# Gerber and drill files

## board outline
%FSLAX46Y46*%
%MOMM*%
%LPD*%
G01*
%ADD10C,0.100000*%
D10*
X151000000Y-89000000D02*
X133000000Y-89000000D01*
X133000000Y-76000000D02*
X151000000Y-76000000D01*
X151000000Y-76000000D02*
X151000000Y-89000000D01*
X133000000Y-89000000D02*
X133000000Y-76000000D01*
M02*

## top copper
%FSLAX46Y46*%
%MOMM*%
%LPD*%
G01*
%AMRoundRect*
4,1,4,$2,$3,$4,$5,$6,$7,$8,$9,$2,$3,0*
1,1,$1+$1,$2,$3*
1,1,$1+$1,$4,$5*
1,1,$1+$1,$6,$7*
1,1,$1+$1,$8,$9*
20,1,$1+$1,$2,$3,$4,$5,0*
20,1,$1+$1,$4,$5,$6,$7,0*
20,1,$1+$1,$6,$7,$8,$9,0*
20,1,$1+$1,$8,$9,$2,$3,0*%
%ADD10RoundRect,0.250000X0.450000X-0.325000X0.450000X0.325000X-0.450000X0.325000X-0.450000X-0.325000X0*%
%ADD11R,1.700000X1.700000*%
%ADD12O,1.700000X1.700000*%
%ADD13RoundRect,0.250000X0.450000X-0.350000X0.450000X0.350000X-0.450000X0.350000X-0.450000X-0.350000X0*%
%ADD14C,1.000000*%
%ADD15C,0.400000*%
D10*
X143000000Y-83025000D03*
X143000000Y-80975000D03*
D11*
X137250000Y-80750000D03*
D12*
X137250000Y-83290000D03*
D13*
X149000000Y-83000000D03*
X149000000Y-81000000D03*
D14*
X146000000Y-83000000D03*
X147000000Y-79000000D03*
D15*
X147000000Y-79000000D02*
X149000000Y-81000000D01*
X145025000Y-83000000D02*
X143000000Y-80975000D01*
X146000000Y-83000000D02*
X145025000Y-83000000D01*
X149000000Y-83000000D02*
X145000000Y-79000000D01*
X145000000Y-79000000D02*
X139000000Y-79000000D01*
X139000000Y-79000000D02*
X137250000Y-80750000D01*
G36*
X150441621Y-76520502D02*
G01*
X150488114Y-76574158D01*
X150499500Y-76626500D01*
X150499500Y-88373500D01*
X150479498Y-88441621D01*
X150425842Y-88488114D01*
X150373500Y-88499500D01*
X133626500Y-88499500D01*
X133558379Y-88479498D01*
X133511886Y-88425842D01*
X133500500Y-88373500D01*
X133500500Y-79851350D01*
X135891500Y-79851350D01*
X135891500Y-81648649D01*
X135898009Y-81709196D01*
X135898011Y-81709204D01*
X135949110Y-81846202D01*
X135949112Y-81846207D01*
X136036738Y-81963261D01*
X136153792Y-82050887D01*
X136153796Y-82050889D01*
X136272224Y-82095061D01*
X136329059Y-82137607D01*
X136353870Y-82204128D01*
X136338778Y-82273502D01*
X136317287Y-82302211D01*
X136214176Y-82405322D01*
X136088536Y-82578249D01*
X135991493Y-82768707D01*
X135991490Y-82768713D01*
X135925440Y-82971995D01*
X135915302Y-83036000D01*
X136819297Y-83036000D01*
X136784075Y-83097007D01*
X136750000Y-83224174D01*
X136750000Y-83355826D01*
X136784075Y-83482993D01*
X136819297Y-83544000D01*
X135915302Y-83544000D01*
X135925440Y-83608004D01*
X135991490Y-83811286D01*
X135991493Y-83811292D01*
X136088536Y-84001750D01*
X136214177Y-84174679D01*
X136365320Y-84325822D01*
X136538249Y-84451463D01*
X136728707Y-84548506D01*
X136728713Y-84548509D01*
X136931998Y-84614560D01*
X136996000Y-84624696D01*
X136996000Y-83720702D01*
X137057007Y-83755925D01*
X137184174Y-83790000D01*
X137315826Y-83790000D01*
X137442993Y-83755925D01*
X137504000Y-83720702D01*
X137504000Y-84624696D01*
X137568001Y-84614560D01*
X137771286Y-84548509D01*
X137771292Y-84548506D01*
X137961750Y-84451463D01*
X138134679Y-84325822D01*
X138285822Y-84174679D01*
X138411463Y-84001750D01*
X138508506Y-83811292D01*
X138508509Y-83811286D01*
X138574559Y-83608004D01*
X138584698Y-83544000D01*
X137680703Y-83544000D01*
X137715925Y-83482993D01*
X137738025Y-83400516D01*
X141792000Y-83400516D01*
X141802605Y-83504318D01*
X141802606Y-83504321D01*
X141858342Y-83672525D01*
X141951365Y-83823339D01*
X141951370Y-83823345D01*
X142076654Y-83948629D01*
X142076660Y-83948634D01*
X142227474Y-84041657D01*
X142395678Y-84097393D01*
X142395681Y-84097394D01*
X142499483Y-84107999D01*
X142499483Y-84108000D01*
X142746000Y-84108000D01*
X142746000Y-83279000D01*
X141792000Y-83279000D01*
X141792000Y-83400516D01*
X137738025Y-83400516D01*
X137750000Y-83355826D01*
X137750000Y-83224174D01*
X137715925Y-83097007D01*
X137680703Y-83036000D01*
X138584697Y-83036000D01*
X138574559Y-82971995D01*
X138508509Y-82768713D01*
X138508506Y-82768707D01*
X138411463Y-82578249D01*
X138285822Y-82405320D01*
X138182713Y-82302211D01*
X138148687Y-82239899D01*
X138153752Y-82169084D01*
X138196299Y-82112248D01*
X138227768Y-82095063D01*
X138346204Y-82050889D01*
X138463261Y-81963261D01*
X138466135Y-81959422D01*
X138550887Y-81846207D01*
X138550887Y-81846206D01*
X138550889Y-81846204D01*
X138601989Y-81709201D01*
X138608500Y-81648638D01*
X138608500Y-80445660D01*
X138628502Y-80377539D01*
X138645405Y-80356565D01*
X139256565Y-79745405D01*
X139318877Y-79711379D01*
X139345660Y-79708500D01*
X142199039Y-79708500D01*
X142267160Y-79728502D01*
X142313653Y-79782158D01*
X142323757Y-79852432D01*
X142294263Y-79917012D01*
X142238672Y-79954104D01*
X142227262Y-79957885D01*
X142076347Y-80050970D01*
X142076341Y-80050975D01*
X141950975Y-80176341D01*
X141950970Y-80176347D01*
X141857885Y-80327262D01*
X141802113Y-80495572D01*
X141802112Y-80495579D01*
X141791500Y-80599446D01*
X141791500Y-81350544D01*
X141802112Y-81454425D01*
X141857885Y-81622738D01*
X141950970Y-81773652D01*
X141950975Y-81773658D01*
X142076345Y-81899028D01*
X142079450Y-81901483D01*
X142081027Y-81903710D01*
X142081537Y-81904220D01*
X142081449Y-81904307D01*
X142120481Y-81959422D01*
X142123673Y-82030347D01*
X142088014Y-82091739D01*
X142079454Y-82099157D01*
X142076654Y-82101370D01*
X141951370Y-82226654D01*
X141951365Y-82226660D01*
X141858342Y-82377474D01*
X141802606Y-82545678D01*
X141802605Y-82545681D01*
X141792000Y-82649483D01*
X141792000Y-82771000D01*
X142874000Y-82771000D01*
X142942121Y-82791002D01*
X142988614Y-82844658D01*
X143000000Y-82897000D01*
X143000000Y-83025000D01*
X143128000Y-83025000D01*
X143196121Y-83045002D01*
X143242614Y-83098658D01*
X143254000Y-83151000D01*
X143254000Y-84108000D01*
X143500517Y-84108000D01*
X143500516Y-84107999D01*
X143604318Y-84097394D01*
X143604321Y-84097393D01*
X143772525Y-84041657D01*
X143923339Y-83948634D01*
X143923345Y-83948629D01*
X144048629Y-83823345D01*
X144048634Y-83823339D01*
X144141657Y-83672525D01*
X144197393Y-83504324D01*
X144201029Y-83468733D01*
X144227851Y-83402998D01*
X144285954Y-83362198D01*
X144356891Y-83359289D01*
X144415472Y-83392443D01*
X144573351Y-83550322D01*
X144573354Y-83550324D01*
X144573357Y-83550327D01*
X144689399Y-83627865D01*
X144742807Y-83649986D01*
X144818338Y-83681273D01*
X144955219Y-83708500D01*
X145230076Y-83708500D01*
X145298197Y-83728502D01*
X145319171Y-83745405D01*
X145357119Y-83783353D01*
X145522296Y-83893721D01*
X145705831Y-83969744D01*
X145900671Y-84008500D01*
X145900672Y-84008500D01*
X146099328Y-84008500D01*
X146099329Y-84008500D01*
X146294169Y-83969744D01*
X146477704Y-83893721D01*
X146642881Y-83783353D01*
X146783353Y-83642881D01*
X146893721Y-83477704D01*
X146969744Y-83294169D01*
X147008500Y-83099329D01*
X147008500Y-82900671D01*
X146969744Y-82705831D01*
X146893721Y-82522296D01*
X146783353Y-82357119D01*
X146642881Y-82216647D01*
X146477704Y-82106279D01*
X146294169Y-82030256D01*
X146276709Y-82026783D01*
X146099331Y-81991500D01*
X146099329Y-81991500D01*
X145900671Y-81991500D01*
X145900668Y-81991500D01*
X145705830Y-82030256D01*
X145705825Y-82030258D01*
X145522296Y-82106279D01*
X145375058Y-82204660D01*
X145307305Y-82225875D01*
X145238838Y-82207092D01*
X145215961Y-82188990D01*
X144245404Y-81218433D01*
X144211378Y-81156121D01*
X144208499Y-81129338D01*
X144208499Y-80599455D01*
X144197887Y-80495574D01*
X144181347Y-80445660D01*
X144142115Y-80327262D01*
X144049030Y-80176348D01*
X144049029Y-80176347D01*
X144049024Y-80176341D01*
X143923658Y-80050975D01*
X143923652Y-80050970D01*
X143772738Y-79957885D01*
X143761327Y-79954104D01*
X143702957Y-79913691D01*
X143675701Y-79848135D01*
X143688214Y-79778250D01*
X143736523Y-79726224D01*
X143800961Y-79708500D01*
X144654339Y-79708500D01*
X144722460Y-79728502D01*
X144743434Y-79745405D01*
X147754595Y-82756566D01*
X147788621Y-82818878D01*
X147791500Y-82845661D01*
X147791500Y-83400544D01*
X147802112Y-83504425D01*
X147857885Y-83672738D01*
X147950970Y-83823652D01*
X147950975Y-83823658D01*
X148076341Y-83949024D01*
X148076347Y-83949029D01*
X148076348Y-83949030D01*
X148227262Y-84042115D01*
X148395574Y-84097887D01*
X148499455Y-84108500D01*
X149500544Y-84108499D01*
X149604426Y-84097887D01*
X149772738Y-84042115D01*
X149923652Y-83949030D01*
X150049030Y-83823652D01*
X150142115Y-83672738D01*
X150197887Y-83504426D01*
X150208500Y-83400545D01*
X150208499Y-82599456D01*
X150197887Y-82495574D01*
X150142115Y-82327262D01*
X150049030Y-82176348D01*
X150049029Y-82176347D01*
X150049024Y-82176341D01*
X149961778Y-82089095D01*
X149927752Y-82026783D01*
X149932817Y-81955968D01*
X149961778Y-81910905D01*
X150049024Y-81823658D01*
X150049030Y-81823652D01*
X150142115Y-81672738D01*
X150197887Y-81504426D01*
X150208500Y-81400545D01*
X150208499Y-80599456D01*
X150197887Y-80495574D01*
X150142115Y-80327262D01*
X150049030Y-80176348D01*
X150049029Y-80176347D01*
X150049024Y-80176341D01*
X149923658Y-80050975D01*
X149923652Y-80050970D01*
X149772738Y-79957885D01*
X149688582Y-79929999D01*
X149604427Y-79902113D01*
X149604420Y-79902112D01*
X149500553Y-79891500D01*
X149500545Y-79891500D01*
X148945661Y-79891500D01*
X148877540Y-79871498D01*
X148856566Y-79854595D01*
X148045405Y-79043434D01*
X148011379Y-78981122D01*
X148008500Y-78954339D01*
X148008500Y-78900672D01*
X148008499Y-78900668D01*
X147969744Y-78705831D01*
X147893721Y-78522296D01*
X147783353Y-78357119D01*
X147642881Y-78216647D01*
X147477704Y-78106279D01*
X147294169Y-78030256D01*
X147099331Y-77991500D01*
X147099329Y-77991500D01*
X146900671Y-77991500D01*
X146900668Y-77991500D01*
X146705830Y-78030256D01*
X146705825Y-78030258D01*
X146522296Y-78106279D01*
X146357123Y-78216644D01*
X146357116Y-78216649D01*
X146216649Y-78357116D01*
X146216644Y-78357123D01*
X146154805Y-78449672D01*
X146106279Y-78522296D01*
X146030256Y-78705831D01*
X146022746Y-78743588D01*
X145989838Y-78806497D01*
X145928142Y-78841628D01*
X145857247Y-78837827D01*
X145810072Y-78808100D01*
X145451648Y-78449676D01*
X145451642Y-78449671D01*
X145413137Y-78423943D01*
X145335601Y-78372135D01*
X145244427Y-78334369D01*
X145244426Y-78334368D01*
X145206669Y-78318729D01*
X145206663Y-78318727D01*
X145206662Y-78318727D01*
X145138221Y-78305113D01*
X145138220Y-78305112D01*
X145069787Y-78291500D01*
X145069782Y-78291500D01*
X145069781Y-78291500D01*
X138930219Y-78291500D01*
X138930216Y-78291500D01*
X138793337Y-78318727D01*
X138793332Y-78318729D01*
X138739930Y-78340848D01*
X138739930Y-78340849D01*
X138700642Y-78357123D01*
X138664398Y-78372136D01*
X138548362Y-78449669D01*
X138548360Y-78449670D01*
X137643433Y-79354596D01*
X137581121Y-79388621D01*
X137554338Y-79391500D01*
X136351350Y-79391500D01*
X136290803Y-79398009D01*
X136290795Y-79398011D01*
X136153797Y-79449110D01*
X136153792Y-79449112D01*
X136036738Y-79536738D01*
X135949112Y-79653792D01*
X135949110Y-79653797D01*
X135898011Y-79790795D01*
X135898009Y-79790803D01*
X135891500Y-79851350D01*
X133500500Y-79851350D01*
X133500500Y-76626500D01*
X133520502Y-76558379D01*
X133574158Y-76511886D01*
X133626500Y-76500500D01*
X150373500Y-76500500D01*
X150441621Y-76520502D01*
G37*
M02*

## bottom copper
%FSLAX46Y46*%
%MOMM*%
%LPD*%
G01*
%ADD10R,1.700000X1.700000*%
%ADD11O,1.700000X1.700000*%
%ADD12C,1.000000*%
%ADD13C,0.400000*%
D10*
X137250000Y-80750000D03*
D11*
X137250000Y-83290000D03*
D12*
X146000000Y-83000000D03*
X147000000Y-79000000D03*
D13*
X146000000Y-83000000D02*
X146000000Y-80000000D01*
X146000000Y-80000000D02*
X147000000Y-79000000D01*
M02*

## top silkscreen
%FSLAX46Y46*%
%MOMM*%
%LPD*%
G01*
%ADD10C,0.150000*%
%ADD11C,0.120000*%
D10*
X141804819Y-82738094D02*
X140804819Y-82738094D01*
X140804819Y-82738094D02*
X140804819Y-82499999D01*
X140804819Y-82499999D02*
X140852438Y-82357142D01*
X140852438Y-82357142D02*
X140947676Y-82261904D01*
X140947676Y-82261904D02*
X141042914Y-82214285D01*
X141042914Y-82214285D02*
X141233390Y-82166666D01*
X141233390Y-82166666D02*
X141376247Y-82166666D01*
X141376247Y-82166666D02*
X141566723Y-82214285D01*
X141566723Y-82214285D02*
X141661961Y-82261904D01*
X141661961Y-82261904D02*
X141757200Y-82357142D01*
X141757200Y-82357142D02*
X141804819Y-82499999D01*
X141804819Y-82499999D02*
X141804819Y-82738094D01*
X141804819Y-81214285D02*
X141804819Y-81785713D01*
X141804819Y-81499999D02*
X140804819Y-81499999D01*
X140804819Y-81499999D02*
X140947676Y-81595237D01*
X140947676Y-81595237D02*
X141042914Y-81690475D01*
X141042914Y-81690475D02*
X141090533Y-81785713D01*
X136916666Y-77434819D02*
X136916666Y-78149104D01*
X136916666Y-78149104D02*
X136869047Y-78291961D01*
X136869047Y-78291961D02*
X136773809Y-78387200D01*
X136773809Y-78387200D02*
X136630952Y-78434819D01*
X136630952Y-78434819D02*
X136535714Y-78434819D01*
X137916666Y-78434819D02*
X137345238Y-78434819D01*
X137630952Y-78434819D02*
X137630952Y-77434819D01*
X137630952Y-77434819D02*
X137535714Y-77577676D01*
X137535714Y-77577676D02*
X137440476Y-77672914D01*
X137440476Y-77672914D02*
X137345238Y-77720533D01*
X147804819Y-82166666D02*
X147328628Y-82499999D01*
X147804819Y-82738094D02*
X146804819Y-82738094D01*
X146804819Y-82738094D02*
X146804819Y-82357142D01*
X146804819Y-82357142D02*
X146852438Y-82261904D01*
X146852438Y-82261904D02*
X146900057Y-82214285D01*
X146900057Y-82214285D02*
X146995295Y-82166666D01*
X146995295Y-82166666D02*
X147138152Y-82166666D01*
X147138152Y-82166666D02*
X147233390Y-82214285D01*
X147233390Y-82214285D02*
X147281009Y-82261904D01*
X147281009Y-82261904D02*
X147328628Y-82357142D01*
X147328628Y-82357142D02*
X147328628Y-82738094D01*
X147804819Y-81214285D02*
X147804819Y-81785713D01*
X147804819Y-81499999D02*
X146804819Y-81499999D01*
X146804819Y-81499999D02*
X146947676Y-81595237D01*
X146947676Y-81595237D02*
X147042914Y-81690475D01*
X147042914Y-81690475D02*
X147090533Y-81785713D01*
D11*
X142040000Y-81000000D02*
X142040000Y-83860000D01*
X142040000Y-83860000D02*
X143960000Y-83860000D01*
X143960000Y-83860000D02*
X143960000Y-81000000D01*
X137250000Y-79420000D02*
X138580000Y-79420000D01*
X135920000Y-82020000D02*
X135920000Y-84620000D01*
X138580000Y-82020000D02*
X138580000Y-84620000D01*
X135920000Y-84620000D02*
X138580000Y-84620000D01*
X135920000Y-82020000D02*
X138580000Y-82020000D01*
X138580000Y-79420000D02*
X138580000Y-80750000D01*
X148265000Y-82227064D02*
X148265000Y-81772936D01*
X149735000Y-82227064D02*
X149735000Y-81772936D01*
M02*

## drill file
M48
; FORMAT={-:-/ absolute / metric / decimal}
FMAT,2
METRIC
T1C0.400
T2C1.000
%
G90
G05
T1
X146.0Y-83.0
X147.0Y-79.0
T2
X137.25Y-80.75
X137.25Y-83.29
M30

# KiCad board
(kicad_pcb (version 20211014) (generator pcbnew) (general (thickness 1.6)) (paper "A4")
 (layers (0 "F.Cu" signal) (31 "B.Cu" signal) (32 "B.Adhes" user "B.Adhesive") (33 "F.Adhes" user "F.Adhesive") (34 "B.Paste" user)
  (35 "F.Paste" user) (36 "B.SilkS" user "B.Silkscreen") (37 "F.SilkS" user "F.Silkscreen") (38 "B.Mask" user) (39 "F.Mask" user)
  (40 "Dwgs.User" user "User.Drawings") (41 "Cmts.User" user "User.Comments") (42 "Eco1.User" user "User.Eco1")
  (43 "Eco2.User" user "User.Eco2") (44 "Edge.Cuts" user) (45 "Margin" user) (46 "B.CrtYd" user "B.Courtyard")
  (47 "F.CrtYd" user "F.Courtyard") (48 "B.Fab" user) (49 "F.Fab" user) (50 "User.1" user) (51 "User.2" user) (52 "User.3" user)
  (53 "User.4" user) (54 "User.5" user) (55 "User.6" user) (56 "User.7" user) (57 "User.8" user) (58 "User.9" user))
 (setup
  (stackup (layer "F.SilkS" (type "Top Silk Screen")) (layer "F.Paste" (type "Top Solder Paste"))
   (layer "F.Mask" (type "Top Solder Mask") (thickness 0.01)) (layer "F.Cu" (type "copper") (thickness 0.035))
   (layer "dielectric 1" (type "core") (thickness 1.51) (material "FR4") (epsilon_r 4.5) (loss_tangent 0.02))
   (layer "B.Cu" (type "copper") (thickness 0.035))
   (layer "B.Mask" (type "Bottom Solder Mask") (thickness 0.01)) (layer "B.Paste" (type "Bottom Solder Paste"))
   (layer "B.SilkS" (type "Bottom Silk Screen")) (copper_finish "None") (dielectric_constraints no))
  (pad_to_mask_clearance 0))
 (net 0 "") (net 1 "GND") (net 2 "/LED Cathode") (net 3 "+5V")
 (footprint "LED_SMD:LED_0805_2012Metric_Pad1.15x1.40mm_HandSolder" (layer "F.Cu") (at 143 82 90)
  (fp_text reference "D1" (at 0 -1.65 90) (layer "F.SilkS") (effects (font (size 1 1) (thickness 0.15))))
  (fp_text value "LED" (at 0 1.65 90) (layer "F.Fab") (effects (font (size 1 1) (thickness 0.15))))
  (fp_line (start 1 -0.96) (end -1.86 -0.96) (layer "F.SilkS") (width 0.12))
  (fp_line (start -1.86 -0.96) (end -1.86 0.96) (layer "F.SilkS") (width 0.12))
  (fp_line (start -1.86 0.96) (end 1 0.96) (layer "F.SilkS") (width 0.12))
  (pad "1" smd roundrect (at -1.025 0 90) (size 1.15 1.4) (layers "F.Cu" "F.Paste" "F.Mask") (roundrect_rratio 0.2173913043) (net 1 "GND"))
  (pad "2" smd roundrect (at 1.025 0 90) (size 1.15 1.4) (layers "F.Cu" "F.Paste" "F.Mask") (roundrect_rratio 0.2173913043)
   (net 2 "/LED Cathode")))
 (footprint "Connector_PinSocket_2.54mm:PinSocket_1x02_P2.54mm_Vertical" (layer "F.Cu") (at 137.25 80.75)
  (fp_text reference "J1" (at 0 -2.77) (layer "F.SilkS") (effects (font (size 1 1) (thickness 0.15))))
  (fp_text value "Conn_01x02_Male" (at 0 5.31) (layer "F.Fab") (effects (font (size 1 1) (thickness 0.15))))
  (fp_line (start 0 -1.33) (end 1.33 -1.33) (layer "F.SilkS") (width 0.12))
  (fp_line (start -1.33 1.27) (end -1.33 3.87) (layer "F.SilkS") (width 0.12))
  (fp_line (start 1.33 1.27) (end 1.33 3.87) (layer "F.SilkS") (width 0.12))
  (fp_line (start -1.33 3.87) (end 1.33 3.87) (layer "F.SilkS") (width 0.12))
  (fp_line (start -1.33 1.27) (end 1.33 1.27) (layer "F.SilkS") (width 0.12))
  (fp_line (start 1.33 -1.33) (end 1.33 0) (layer "F.SilkS") (width 0.12))
  (pad "1" thru_hole rect (at 0 0) (size 1.7 1.7) (drill 1) (layers *.Cu *.Mask) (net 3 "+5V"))
  (pad "2" thru_hole oval (at 0 2.54) (size 1.7 1.7) (drill 1) (layers *.Cu *.Mask) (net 1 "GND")))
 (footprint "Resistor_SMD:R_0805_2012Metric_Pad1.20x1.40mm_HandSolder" (layer "F.Cu") (at 149 82 90)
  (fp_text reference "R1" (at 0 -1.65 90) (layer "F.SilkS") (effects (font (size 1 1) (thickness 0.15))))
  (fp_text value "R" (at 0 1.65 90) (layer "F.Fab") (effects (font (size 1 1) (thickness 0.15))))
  (fp_line (start -0.227064 -0.735) (end 0.227064 -0.735) (layer "F.SilkS") (width 0.12))
  (fp_line (start -0.227064 0.735) (end 0.227064 0.735) (layer "F.SilkS") (width 0.12))
  (pad "1" smd roundrect (at -1 0 90) (size 1.2 1.4) (layers "F.Cu" "F.Paste" "F.Mask") (roundrect_rratio 0.2083333333) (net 3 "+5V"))
  (pad "2" smd roundrect (at 1 0 90) (size 1.2 1.4) (layers "F.Cu" "F.Paste" "F.Mask") (roundrect_rratio 0.2083333333)
   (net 2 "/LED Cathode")))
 (gr_line (start 151 89) (end 133 89) (layer "Edge.Cuts") (width 0.1))
 (gr_line (start 133 76) (end 151 76) (layer "Edge.Cuts") (width 0.1))
 (gr_line (start 151 76) (end 151 89) (layer "Edge.Cuts") (width 0.1))
 (gr_line (start 133 89) (end 133 76) (layer "Edge.Cuts") (width 0.1))
 (segment (start 147 79) (end 149 81) (width 0.4) (layer "F.Cu") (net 2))
 (segment (start 145.025 83) (end 143 80.975) (width 0.4) (layer "F.Cu") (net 2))
 (segment (start 146 83) (end 145.025 83) (width 0.4) (layer "F.Cu") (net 2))
 (via (at 146 83) (size 1) (drill 0.4) (layers "F.Cu" "B.Cu") (free) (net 2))
 (via (at 147 79) (size 1) (drill 0.4) (layers "F.Cu" "B.Cu") (free) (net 2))
 (segment (start 146 83) (end 146 80) (width 0.4) (layer "B.Cu") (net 2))
 (segment (start 146 80) (end 147 79) (width 0.4) (layer "B.Cu") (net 2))
 (segment (start 149 83) (end 145 79) (width 0.4) (layer "F.Cu") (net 3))
 (segment (start 145 79) (end 139 79) (width 0.4) (layer "F.Cu") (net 3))
 (segment (start 139 79) (end 137.25 80.75) (width 0.4) (layer "F.Cu") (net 3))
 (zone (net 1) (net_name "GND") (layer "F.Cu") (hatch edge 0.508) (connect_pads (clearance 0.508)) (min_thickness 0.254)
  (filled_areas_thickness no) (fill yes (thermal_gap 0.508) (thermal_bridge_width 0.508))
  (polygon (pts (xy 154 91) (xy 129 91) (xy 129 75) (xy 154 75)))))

